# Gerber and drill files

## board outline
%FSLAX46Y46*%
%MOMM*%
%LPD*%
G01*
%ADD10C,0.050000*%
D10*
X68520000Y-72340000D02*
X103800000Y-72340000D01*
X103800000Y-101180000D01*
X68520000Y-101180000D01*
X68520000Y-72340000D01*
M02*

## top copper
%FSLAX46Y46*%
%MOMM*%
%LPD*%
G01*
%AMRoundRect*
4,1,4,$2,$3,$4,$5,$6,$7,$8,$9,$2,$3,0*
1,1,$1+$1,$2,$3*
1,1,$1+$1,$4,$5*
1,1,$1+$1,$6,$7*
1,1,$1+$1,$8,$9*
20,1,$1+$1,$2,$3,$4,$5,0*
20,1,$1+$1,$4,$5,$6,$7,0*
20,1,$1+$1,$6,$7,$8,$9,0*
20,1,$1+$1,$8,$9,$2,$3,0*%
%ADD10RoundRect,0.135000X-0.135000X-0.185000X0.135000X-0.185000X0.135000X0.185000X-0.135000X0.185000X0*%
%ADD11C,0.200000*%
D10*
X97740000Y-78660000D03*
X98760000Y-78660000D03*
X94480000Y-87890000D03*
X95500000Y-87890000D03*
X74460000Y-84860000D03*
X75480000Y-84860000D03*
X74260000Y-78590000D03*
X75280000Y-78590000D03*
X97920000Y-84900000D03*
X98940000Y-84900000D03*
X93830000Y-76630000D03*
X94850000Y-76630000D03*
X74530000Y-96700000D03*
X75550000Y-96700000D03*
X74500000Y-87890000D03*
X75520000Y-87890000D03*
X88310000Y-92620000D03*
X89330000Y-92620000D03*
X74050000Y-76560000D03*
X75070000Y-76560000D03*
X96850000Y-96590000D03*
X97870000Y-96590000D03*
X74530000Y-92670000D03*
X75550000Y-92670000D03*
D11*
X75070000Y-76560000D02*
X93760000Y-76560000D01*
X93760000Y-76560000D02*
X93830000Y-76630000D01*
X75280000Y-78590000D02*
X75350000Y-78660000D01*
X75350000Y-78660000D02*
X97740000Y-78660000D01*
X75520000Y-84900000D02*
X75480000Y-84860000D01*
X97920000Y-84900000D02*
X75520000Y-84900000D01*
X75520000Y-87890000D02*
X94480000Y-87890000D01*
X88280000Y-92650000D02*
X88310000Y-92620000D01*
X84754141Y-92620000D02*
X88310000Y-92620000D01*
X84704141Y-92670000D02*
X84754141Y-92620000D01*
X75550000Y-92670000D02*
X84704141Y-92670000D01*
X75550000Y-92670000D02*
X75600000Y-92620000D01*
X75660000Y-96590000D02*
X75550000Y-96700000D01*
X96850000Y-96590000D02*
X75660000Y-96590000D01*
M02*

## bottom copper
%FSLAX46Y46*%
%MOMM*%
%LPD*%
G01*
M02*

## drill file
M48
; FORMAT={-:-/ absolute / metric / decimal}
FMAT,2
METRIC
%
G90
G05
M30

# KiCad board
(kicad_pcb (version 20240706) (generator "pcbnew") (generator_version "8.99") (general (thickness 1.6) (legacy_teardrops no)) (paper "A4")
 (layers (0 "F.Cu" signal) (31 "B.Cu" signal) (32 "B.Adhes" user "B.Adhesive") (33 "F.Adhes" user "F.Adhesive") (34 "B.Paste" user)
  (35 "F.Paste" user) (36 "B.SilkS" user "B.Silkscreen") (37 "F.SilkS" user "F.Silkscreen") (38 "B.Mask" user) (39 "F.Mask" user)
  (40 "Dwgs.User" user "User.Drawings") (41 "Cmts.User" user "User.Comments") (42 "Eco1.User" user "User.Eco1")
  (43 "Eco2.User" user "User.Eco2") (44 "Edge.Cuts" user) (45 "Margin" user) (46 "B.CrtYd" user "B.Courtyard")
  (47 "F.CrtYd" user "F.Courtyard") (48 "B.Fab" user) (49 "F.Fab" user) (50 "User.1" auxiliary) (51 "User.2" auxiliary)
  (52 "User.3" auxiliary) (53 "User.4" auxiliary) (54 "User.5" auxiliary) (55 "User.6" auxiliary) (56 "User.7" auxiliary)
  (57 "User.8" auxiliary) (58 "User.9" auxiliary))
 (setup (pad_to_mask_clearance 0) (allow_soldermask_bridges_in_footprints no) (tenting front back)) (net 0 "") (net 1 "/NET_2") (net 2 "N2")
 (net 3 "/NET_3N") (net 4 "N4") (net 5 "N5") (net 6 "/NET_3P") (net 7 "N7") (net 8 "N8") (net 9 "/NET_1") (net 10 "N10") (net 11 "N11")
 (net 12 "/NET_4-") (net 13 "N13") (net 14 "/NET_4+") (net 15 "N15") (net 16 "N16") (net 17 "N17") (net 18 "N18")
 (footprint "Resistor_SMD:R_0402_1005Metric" (layer "F.Cu") (at 98.25 78.66)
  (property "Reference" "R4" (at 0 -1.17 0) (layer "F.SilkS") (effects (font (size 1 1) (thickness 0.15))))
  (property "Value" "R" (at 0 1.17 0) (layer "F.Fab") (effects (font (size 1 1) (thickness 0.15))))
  (pad "1" smd roundrect (at -0.51 0) (size 0.54 0.64) (layers "F.Cu" "F.Paste" "F.Mask") (roundrect_rratio 0.25) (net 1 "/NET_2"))
  (pad "2" smd roundrect (at 0.51 0) (size 0.54 0.64) (layers "F.Cu" "F.Paste" "F.Mask") (roundrect_rratio 0.25) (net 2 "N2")))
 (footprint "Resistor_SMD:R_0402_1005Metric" (layer "F.Cu") (at 94.99 87.89)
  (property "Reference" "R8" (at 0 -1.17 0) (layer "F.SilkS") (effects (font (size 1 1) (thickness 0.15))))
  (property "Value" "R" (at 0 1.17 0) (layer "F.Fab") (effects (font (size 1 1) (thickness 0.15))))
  (pad "1" smd roundrect (at -0.51 0) (size 0.54 0.64) (layers "F.Cu" "F.Paste" "F.Mask") (roundrect_rratio 0.25) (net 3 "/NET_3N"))
  (pad "2" smd roundrect (at 0.51 0) (size 0.54 0.64) (layers "F.Cu" "F.Paste" "F.Mask") (roundrect_rratio 0.25) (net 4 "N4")))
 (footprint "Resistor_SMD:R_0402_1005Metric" (layer "F.Cu") (at 74.97 84.86)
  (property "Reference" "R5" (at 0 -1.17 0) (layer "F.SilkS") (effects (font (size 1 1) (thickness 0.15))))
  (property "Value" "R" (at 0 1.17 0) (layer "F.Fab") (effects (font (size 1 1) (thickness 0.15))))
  (pad "1" smd roundrect (at -0.51 0) (size 0.54 0.64) (layers "F.Cu" "F.Paste" "F.Mask") (roundrect_rratio 0.25) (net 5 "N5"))
  (pad "2" smd roundrect (at 0.51 0) (size 0.54 0.64) (layers "F.Cu" "F.Paste" "F.Mask") (roundrect_rratio 0.25) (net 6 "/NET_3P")))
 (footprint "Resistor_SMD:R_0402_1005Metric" (layer "F.Cu") (at 74.77 78.59)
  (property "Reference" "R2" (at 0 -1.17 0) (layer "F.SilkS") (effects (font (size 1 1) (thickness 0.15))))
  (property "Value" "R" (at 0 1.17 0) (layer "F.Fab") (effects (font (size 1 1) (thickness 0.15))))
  (pad "1" smd roundrect (at -0.51 0) (size 0.54 0.64) (layers "F.Cu" "F.Paste" "F.Mask") (roundrect_rratio 0.25) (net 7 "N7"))
  (pad "2" smd roundrect (at 0.51 0) (size 0.54 0.64) (layers "F.Cu" "F.Paste" "F.Mask") (roundrect_rratio 0.25) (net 1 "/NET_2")))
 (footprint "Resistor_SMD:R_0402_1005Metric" (layer "F.Cu") (at 98.43 84.9)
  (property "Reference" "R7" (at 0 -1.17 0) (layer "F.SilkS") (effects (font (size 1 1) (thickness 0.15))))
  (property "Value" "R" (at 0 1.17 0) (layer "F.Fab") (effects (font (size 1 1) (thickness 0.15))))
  (pad "1" smd roundrect (at -0.51 0) (size 0.54 0.64) (layers "F.Cu" "F.Paste" "F.Mask") (roundrect_rratio 0.25) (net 6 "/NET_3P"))
  (pad "2" smd roundrect (at 0.51 0) (size 0.54 0.64) (layers "F.Cu" "F.Paste" "F.Mask") (roundrect_rratio 0.25) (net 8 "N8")))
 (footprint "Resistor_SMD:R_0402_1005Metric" (layer "F.Cu") (at 94.34 76.63)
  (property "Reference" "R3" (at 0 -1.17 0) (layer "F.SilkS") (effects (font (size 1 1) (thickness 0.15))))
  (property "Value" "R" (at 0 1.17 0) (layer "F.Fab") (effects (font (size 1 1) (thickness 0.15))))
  (pad "1" smd roundrect (at -0.51 0) (size 0.54 0.64) (layers "F.Cu" "F.Paste" "F.Mask") (roundrect_rratio 0.25) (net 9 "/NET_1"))
  (pad "2" smd roundrect (at 0.51 0) (size 0.54 0.64) (layers "F.Cu" "F.Paste" "F.Mask") (roundrect_rratio 0.25) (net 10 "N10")))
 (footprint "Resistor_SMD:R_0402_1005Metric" (layer "F.Cu") (at 75.04 96.7)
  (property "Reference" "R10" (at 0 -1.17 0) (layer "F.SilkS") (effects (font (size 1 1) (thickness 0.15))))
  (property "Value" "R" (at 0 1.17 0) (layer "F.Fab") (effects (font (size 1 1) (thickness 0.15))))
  (pad "1" smd roundrect (at -0.51 0) (size 0.54 0.64) (layers "F.Cu" "F.Paste" "F.Mask") (roundrect_rratio 0.25) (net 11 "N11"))
  (pad "2" smd roundrect (at 0.51 0) (size 0.54 0.64) (layers "F.Cu" "F.Paste" "F.Mask") (roundrect_rratio 0.25) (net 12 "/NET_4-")))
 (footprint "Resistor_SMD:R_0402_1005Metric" (layer "F.Cu") (at 75.01 87.89)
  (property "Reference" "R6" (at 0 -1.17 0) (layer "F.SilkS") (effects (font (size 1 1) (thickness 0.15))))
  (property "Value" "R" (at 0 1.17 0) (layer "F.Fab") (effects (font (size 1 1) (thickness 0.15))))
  (pad "1" smd roundrect (at -0.51 0) (size 0.54 0.64) (layers "F.Cu" "F.Paste" "F.Mask") (roundrect_rratio 0.25) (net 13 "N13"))
  (pad "2" smd roundrect (at 0.51 0) (size 0.54 0.64) (layers "F.Cu" "F.Paste" "F.Mask") (roundrect_rratio 0.25) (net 3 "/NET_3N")))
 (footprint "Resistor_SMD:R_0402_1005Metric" (layer "F.Cu") (at 88.82 92.62)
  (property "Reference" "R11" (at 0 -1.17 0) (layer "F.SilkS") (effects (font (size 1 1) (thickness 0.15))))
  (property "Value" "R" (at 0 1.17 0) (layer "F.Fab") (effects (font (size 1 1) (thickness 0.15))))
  (pad "1" smd roundrect (at -0.51 0) (size 0.54 0.64) (layers "F.Cu" "F.Paste" "F.Mask") (roundrect_rratio 0.25) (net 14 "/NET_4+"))
  (pad "2" smd roundrect (at 0.51 0) (size 0.54 0.64) (layers "F.Cu" "F.Paste" "F.Mask") (roundrect_rratio 0.25) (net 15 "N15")))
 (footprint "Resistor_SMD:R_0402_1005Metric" (layer "F.Cu") (at 74.56 76.56)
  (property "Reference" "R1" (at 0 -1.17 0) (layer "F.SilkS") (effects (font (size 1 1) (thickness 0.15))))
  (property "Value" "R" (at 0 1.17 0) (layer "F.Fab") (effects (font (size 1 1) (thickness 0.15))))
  (pad "1" smd roundrect (at -0.51 0) (size 0.54 0.64) (layers "F.Cu" "F.Paste" "F.Mask") (roundrect_rratio 0.25) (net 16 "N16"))
  (pad "2" smd roundrect (at 0.51 0) (size 0.54 0.64) (layers "F.Cu" "F.Paste" "F.Mask") (roundrect_rratio 0.25) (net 9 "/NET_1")))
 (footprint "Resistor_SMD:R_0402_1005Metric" (layer "F.Cu") (at 97.36 96.59)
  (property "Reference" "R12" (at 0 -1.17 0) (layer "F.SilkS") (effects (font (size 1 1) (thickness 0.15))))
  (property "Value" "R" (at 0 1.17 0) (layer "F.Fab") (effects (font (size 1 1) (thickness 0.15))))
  (pad "1" smd roundrect (at -0.51 0) (size 0.54 0.64) (layers "F.Cu" "F.Paste" "F.Mask") (roundrect_rratio 0.25) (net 12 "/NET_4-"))
  (pad "2" smd roundrect (at 0.51 0) (size 0.54 0.64) (layers "F.Cu" "F.Paste" "F.Mask") (roundrect_rratio 0.25) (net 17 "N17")))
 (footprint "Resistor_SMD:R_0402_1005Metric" (layer "F.Cu") (at 75.04 92.67)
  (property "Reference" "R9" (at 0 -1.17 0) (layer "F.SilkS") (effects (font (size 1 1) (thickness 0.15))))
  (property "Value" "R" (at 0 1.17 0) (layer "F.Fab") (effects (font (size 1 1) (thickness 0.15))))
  (pad "1" smd roundrect (at -0.51 0) (size 0.54 0.64) (layers "F.Cu" "F.Paste" "F.Mask") (roundrect_rratio 0.25) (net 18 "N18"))
  (pad "2" smd roundrect (at 0.51 0) (size 0.54 0.64) (layers "F.Cu" "F.Paste" "F.Mask") (roundrect_rratio 0.25) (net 14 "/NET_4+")))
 (gr_rect (start 68.52 72.34) (end 103.8 101.18) (stroke (width 0.05) (type default)) (fill none) (layer "Edge.Cuts"))
 (segment (start 75.07 76.56) (end 93.76 76.56) (width 0.2) (layer "F.Cu") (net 9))
 (segment (start 93.76 76.56) (end 93.83 76.63) (width 0.2) (layer "F.Cu") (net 9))
 (segment (start 75.28 78.59) (end 75.35 78.66) (width 0.2) (layer "F.Cu") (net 1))
 (segment (start 75.35 78.66) (end 97.74 78.66) (width 0.2) (layer "F.Cu") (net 1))
 (segment (start 75.52 84.9) (end 75.48 84.86) (width 0.2) (layer "F.Cu") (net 6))
 (segment (start 97.92 84.9) (end 75.52 84.9) (width 0.2) (layer "F.Cu") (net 6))
 (segment (start 75.52 87.89) (end 94.48 87.89) (width 0.2) (layer "F.Cu") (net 3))
 (segment (start 88.28 92.65) (end 88.31 92.62) (width 0.2) (layer "F.Cu") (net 14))
 (segment (start 84.754141 92.62) (end 88.31 92.62) (width 0.2) (layer "F.Cu") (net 14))
 (segment (start 84.704141 92.67) (end 84.754141 92.62) (width 0.2) (layer "F.Cu") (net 14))
 (segment (start 75.55 92.67) (end 84.704141 92.67) (width 0.2) (layer "F.Cu") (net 14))
 (segment (start 75.55 92.67) (end 75.6 92.62) (width 0.2) (layer "F.Cu") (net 14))
 (segment (start 75.66 96.59) (end 75.55 96.7) (width 0.2) (layer "F.Cu") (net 12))
 (segment (start 96.85 96.59) (end 75.66 96.59) (width 0.2) (layer "F.Cu") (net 12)))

